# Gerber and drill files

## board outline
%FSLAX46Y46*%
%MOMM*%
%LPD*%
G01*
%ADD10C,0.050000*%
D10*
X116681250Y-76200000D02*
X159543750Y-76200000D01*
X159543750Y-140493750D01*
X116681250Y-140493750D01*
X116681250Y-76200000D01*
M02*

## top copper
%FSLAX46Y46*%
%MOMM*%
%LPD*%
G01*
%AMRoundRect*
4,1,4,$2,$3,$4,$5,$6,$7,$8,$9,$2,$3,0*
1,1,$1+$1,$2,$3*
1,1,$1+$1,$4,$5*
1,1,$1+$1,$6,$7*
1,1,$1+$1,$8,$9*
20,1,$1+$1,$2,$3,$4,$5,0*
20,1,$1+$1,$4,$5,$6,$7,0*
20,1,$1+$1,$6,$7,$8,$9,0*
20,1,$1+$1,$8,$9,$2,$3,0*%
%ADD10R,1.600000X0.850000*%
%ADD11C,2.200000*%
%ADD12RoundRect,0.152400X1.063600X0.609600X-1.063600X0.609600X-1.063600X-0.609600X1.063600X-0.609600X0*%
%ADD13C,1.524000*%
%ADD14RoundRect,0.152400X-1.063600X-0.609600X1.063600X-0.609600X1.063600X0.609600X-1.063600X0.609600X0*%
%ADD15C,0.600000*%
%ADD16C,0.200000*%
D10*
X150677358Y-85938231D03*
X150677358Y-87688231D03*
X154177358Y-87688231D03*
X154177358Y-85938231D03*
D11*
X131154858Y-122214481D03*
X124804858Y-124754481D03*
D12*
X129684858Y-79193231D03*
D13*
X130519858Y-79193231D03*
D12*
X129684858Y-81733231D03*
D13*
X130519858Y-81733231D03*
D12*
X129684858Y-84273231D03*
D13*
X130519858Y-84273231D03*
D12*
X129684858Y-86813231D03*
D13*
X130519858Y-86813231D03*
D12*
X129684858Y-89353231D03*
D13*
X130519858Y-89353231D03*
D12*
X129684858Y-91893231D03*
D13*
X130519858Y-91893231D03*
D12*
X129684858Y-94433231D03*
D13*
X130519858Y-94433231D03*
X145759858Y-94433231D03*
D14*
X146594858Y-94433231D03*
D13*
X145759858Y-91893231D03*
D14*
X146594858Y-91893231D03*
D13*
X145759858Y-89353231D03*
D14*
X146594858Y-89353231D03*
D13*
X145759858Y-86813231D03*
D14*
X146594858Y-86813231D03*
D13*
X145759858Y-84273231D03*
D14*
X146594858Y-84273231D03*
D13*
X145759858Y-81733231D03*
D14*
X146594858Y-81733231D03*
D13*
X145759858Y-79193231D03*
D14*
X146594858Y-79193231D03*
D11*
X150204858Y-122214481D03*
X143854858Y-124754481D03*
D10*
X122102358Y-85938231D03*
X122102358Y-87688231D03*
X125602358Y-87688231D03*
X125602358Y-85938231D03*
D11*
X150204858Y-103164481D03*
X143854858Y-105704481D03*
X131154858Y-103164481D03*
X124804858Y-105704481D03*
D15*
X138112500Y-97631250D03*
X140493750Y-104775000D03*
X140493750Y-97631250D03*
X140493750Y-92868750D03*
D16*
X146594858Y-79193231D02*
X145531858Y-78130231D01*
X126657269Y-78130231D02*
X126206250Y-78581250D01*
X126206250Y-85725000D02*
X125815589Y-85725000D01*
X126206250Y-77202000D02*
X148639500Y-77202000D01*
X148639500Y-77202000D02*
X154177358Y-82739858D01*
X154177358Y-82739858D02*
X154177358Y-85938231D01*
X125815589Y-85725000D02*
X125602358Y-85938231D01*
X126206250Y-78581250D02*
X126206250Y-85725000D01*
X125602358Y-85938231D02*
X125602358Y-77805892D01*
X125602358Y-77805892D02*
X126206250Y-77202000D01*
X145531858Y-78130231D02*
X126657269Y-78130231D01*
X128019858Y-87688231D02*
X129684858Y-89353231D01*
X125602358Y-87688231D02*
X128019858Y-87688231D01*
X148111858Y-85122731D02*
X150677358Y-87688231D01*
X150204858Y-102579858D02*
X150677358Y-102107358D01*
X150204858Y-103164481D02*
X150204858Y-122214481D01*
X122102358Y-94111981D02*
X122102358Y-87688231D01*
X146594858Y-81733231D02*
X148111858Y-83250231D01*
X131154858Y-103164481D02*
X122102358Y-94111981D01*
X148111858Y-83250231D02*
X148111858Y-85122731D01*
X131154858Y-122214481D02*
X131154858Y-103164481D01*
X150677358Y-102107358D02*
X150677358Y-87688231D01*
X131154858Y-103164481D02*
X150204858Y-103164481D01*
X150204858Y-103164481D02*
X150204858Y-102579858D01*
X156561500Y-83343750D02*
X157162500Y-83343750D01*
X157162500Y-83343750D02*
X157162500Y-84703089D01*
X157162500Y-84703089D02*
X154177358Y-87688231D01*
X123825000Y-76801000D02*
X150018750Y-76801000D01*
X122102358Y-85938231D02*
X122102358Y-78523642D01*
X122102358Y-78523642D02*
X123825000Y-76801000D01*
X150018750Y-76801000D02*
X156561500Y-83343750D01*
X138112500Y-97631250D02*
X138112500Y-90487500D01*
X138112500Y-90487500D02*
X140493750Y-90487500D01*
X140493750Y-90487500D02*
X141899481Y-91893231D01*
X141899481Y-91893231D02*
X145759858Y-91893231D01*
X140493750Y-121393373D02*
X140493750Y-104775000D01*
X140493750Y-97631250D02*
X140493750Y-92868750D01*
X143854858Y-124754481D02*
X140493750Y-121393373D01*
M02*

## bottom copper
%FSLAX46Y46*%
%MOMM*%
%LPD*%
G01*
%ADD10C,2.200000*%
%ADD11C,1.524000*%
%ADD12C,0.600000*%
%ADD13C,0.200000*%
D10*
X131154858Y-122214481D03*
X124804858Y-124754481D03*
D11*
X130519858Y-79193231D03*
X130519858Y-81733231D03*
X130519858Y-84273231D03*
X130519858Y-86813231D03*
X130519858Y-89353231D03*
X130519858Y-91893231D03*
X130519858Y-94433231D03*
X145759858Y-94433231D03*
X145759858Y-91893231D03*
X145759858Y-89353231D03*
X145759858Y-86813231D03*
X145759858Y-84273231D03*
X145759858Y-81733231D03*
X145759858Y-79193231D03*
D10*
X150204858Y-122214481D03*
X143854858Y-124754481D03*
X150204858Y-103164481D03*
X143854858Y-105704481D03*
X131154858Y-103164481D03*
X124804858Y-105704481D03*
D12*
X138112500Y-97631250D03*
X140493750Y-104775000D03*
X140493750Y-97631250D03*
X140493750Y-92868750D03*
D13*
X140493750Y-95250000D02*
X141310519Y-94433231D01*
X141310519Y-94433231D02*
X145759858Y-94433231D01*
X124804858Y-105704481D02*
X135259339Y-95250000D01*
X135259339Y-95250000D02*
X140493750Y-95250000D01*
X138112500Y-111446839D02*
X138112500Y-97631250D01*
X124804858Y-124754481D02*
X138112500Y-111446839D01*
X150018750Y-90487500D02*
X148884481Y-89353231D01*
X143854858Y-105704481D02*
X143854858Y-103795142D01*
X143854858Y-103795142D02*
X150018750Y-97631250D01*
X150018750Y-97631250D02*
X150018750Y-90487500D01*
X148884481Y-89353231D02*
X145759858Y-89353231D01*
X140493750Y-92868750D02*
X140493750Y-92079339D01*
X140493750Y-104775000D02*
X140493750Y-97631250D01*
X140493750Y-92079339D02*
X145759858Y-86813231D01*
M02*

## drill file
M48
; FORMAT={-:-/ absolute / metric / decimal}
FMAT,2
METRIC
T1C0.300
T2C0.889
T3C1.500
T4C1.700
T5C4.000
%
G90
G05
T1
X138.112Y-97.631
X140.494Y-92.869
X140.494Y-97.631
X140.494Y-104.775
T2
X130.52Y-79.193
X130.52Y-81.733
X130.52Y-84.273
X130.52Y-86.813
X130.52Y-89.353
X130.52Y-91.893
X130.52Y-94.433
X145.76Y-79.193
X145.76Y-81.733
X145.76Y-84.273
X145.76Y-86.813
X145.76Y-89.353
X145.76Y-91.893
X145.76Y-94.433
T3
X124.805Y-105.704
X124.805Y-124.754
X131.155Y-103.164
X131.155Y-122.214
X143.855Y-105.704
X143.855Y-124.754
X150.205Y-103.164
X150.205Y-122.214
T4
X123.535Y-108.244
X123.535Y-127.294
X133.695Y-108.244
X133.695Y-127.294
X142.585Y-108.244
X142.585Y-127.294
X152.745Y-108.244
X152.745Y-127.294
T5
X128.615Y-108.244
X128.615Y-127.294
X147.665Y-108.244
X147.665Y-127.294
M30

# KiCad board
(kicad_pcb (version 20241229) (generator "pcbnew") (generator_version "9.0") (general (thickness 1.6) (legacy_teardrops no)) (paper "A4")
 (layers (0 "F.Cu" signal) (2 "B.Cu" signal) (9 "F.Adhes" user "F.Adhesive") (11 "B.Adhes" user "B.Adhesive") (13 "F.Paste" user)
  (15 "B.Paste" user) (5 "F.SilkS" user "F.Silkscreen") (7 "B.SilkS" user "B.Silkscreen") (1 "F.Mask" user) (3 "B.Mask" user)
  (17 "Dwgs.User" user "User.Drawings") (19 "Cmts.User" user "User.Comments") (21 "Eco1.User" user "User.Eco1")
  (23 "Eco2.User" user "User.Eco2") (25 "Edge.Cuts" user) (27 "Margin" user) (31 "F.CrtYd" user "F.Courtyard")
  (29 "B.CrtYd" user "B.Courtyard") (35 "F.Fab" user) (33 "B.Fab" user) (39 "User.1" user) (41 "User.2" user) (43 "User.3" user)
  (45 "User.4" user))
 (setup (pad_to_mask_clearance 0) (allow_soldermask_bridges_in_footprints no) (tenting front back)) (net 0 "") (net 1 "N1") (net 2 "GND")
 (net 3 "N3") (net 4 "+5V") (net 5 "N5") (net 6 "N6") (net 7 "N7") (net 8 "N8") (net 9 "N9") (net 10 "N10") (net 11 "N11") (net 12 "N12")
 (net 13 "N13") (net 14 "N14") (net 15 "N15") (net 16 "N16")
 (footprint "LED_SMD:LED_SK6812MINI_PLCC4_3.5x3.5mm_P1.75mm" (layer "F.Cu") (at 152.427358 86.813231)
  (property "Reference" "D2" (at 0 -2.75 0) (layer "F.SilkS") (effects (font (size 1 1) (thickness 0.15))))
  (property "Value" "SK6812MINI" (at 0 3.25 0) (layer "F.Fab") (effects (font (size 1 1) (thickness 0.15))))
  (pad "1" smd rect (at -1.75 -0.875) (size 1.6 0.85) (layers "F.Cu" "F.Mask" "F.Paste") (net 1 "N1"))
  (pad "2" smd rect (at -1.75 0.875) (size 1.6 0.85) (layers "F.Cu" "F.Mask" "F.Paste") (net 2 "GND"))
  (pad "3" smd rect (at 1.75 0.875) (size 1.6 0.85) (layers "F.Cu" "F.Mask" "F.Paste") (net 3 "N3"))
  (pad "4" smd rect (at 1.75 -0.875) (size 1.6 0.85) (layers "F.Cu" "F.Mask" "F.Paste") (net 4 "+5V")))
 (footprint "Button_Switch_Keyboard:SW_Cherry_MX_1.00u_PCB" (layer "F.Cu") (at 131.154858 122.214481)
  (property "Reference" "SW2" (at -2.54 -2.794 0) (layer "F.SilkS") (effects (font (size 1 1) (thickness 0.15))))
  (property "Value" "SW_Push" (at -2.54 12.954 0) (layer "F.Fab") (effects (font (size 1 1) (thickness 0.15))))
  (pad "" np_thru_hole circle (at -7.62 5.08) (size 1.7 1.7) (drill 1.7) (layers "*.Cu" "*.Mask"))
  (pad "" np_thru_hole circle (at -2.54 5.08) (size 4 4) (drill 4) (layers "*.Cu" "*.Mask"))
  (pad "" np_thru_hole circle (at 2.54 5.08) (size 1.7 1.7) (drill 1.7) (layers "*.Cu" "*.Mask"))
  (pad "1" thru_hole circle (at 0 0) (size 2.2 2.2) (drill 1.5) (layers "*.Cu" "*.Mask") (remove_unused_layers no) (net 2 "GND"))
  (pad "2" thru_hole circle (at -6.35 2.54) (size 2.2 2.2) (drill 1.5) (layers "*.Cu" "*.Mask") (remove_unused_layers no) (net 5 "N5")))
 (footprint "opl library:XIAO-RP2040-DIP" (layer "F.Cu") (at 138.139858 86.813231)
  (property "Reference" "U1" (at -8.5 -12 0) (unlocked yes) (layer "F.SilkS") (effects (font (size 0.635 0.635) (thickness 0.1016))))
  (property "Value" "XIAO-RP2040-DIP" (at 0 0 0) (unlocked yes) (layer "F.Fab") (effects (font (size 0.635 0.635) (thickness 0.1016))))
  (pad "1" smd roundrect (at -8.455 -7.62 180) (size 2.432 1.524) (layers "F.Cu" "F.Mask") (roundrect_rratio 0.1) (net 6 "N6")
   (thermal_bridge_angle 45))
  (pad "1" thru_hole circle (at -7.62 -7.62 180) (size 1.524 1.524) (drill 0.889) (layers "*.Cu" "*.Mask") (remove_unused_layers no)
   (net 6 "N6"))
  (pad "2" smd roundrect (at -8.455 -5.08 180) (size 2.432 1.524) (layers "F.Cu" "F.Mask") (roundrect_rratio 0.1) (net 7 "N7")
   (thermal_bridge_angle 45))
  (pad "2" thru_hole circle (at -7.62 -5.08 180) (size 1.524 1.524) (drill 0.889) (layers "*.Cu" "*.Mask") (remove_unused_layers no)
   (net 7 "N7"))
  (pad "3" smd roundrect (at -8.455 -2.54 180) (size 2.432 1.524) (layers "F.Cu" "F.Mask") (roundrect_rratio 0.1) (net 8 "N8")
   (thermal_bridge_angle 45))
  (pad "3" thru_hole circle (at -7.62 -2.54 180) (size 1.524 1.524) (drill 0.889) (layers "*.Cu" "*.Mask") (remove_unused_layers no)
   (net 8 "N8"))
  (pad "4" smd roundrect (at -8.455 0 180) (size 2.432 1.524) (layers "F.Cu" "F.Mask") (roundrect_rratio 0.1) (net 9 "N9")
   (thermal_bridge_angle 45))
  (pad "4" thru_hole circle (at -7.62 0 180) (size 1.524 1.524) (drill 0.889) (layers "*.Cu" "*.Mask") (remove_unused_layers no)
   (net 9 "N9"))
  (pad "5" smd roundrect (at -8.455 2.54 180) (size 2.432 1.524) (layers "F.Cu" "F.Mask") (roundrect_rratio 0.1) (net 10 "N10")
   (thermal_bridge_angle 45))
  (pad "5" thru_hole circle (at -7.62 2.54 180) (size 1.524 1.524) (drill 0.889) (layers "*.Cu" "*.Mask") (remove_unused_layers no)
   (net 10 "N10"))
  (pad "6" smd roundrect (at -8.455 5.08 180) (size 2.432 1.524) (layers "F.Cu" "F.Mask") (roundrect_rratio 0.1) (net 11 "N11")
   (thermal_bridge_angle 45))
  (pad "6" thru_hole circle (at -7.62 5.08 180) (size 1.524 1.524) (drill 0.889) (layers "*.Cu" "*.Mask") (remove_unused_layers no)
   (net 11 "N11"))
  (pad "7" smd roundrect (at -8.455 7.62 180) (size 2.432 1.524) (layers "F.Cu" "F.Mask") (roundrect_rratio 0.1) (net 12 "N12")
   (thermal_bridge_angle 45))
  (pad "7" thru_hole circle (at -7.62 7.62 180) (size 1.524 1.524) (drill 0.889) (layers "*.Cu" "*.Mask") (remove_unused_layers no)
   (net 12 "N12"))
  (pad "8" thru_hole circle (at 7.62 7.62) (size 1.524 1.524) (drill 0.889) (layers "*.Cu" "*.Mask") (remove_unused_layers no)
   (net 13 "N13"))
  (pad "8" smd roundrect (at 8.455 7.62) (size 2.432 1.524) (layers "F.Cu" "F.Mask") (roundrect_rratio 0.1) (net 13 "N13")
   (thermal_bridge_angle 45))
  (pad "9" thru_hole circle (at 7.62 5.08) (size 1.524 1.524) (drill 0.889) (layers "*.Cu" "*.Mask") (remove_unused_layers no) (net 5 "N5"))
  (pad "9" smd roundrect (at 8.455 5.08) (size 2.432 1.524) (layers "F.Cu" "F.Mask") (roundrect_rratio 0.1) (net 5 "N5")
   (thermal_bridge_angle 45))
  (pad "10" thru_hole circle (at 7.62 2.54) (size 1.524 1.524) (drill 0.889) (layers "*.Cu" "*.Mask") (remove_unused_layers no)
   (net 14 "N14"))
  (pad "10" smd roundrect (at 8.455 2.54) (size 2.432 1.524) (layers "F.Cu" "F.Mask") (roundrect_rratio 0.1) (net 14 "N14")
   (thermal_bridge_angle 45))
  (pad "11" thru_hole circle (at 7.62 0) (size 1.524 1.524) (drill 0.889) (layers "*.Cu" "*.Mask") (remove_unused_layers no) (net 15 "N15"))
  (pad "11" smd roundrect (at 8.455 0) (size 2.432 1.524) (layers "F.Cu" "F.Mask") (roundrect_rratio 0.1) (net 15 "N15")
   (thermal_bridge_angle 45))
  (pad "12" thru_hole circle (at 7.62 -2.54) (size 1.524 1.524) (drill 0.889) (layers "*.Cu" "*.Mask") (remove_unused_layers no)
   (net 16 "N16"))
  (pad "12" smd roundrect (at 8.455 -2.54) (size 2.432 1.524) (layers "F.Cu" "F.Mask") (roundrect_rratio 0.1) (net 16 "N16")
   (thermal_bridge_angle 45))
  (pad "13" thru_hole circle (at 7.62 -5.08) (size 1.524 1.524) (drill 0.889) (layers "*.Cu" "*.Mask") (remove_unused_layers no)
   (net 2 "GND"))
  (pad "13" smd roundrect (at 8.455 -5.08) (size 2.432 1.524) (layers "F.Cu" "F.Mask") (roundrect_rratio 0.1) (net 2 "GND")
   (thermal_bridge_angle 45))
  (pad "14" thru_hole circle (at 7.62 -7.62) (size 1.524 1.524) (drill 0.889) (layers "*.Cu" "*.Mask") (remove_unused_layers no)
   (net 4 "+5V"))
  (pad "14" smd roundrect (at 8.455 -7.62) (size 2.432 1.524) (layers "F.Cu" "F.Mask") (roundrect_rratio 0.1) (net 4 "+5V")
   (thermal_bridge_angle 45)))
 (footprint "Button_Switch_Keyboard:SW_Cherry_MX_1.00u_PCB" (layer "F.Cu") (at 150.204858 122.214481)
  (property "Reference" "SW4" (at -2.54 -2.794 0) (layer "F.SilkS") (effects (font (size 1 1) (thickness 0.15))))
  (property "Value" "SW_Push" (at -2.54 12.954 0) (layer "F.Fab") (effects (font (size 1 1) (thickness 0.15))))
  (pad "" np_thru_hole circle (at -7.62 5.08) (size 1.7 1.7) (drill 1.7) (layers "*.Cu" "*.Mask"))
  (pad "" np_thru_hole circle (at -2.54 5.08) (size 4 4) (drill 4) (layers "*.Cu" "*.Mask"))
  (pad "" np_thru_hole circle (at 2.54 5.08) (size 1.7 1.7) (drill 1.7) (layers "*.Cu" "*.Mask"))
  (pad "1" thru_hole circle (at 0 0) (size 2.2 2.2) (drill 1.5) (layers "*.Cu" "*.Mask") (remove_unused_layers no) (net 2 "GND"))
  (pad "2" thru_hole circle (at -6.35 2.54) (size 2.2 2.2) (drill 1.5) (layers "*.Cu" "*.Mask") (remove_unused_layers no) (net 15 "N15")))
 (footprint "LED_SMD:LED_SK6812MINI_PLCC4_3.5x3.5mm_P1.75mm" (layer "F.Cu") (at 123.852358 86.813231)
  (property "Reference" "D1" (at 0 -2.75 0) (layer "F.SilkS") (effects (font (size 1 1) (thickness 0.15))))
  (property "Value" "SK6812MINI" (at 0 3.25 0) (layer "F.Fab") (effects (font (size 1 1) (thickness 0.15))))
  (pad "1" smd rect (at -1.75 -0.875) (size 1.6 0.85) (layers "F.Cu" "F.Mask" "F.Paste") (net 3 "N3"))
  (pad "2" smd rect (at -1.75 0.875) (size 1.6 0.85) (layers "F.Cu" "F.Mask" "F.Paste") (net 2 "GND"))
  (pad "3" smd rect (at 1.75 0.875) (size 1.6 0.85) (layers "F.Cu" "F.Mask" "F.Paste") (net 10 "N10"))
  (pad "4" smd rect (at 1.75 -0.875) (size 1.6 0.85) (layers "F.Cu" "F.Mask" "F.Paste") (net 4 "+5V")))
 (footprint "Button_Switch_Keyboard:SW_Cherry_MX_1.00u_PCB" (layer "F.Cu") (at 150.204858 103.164481)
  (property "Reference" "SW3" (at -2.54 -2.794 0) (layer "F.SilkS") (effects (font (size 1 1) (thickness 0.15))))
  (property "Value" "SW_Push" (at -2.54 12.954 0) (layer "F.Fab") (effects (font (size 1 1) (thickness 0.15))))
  (pad "" np_thru_hole circle (at -7.62 5.08) (size 1.7 1.7) (drill 1.7) (layers "*.Cu" "*.Mask"))
  (pad "" np_thru_hole circle (at -2.54 5.08) (size 4 4) (drill 4) (layers "*.Cu" "*.Mask"))
  (pad "" np_thru_hole circle (at 2.54 5.08) (size 1.7 1.7) (drill 1.7) (layers "*.Cu" "*.Mask"))
  (pad "1" thru_hole circle (at 0 0) (size 2.2 2.2) (drill 1.5) (layers "*.Cu" "*.Mask") (remove_unused_layers no) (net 2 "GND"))
  (pad "2" thru_hole circle (at -6.35 2.54) (size 2.2 2.2) (drill 1.5) (layers "*.Cu" "*.Mask") (remove_unused_layers no) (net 14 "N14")))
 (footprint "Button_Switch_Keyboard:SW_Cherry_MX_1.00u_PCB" (layer "F.Cu") (at 131.154858 103.164481)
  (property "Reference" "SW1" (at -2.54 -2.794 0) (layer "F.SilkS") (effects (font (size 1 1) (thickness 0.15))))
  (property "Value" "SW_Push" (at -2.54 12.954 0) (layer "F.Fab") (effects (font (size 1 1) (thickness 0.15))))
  (pad "" np_thru_hole circle (at -7.62 5.08) (size 1.7 1.7) (drill 1.7) (layers "*.Cu" "*.Mask"))
  (pad "" np_thru_hole circle (at -2.54 5.08) (size 4 4) (drill 4) (layers "*.Cu" "*.Mask"))
  (pad "" np_thru_hole circle (at 2.54 5.08) (size 1.7 1.7) (drill 1.7) (layers "*.Cu" "*.Mask"))
  (pad "1" thru_hole circle (at 0 0) (size 2.2 2.2) (drill 1.5) (layers "*.Cu" "*.Mask") (remove_unused_layers no) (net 2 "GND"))
  (pad "2" thru_hole circle (at -6.35 2.54) (size 2.2 2.2) (drill 1.5) (layers "*.Cu" "*.Mask") (remove_unused_layers no) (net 13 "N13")))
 (gr_rect (start 116.68125 76.2) (end 159.54375 140.49375) (stroke (width 0.05) (type default)) (fill no) (layer "Edge.Cuts"))
 (segment (start 146.594858 79.193231) (end 145.531858 78.130231) (width 0.2) (layer "F.Cu") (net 4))
 (segment (start 126.657269 78.130231) (end 126.20625 78.58125) (width 0.2) (layer "F.Cu") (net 4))
 (segment (start 126.20625 85.725) (end 125.815589 85.725) (width 0.2) (layer "F.Cu") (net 4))
 (segment (start 126.20625 77.202) (end 148.6395 77.202) (width 0.2) (layer "F.Cu") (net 4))
 (segment (start 148.6395 77.202) (end 154.177358 82.739858) (width 0.2) (layer "F.Cu") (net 4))
 (segment (start 154.177358 82.739858) (end 154.177358 85.938231) (width 0.2) (layer "F.Cu") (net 4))
 (segment (start 125.815589 85.725) (end 125.602358 85.938231) (width 0.2) (layer "F.Cu") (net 4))
 (segment (start 126.20625 78.58125) (end 126.20625 85.725) (width 0.2) (layer "F.Cu") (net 4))
 (segment (start 125.602358 85.938231) (end 125.602358 77.805892) (width 0.2) (layer "F.Cu") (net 4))
 (segment (start 125.602358 77.805892) (end 126.20625 77.202) (width 0.2) (layer "F.Cu") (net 4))
 (segment (start 145.531858 78.130231) (end 126.657269 78.130231) (width 0.2) (layer "F.Cu") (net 4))
 (segment (start 128.019858 87.688231) (end 129.684858 89.353231) (width 0.2) (layer "F.Cu") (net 10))
 (segment (start 125.602358 87.688231) (end 128.019858 87.688231) (width 0.2) (layer "F.Cu") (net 10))
 (segment (start 148.111858 85.122731) (end 150.677358 87.688231) (width 0.2) (layer "F.Cu") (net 2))
 (segment (start 150.204858 102.579858) (end 150.677358 102.107358) (width 0.2) (layer "F.Cu") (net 2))
 (segment (start 150.204858 103.164481) (end 150.204858 122.214481) (width 0.2) (layer "F.Cu") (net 2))
 (segment (start 122.102358 94.111981) (end 122.102358 87.688231) (width 0.2) (layer "F.Cu") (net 2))
 (segment (start 146.594858 81.733231) (end 148.111858 83.250231) (width 0.2) (layer "F.Cu") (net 2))
 (segment (start 131.154858 103.164481) (end 122.102358 94.111981) (width 0.2) (layer "F.Cu") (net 2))
 (segment (start 148.111858 83.250231) (end 148.111858 85.122731) (width 0.2) (layer "F.Cu") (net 2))
 (segment (start 131.154858 122.214481) (end 131.154858 103.164481) (width 0.2) (layer "F.Cu") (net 2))
 (segment (start 150.677358 102.107358) (end 150.677358 87.688231) (width 0.2) (layer "F.Cu") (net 2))
 (segment (start 131.154858 103.164481) (end 150.204858 103.164481) (width 0.2) (layer "F.Cu") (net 2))
 (segment (start 150.204858 103.164481) (end 150.204858 102.579858) (width 0.2) (layer "F.Cu") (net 2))
 (segment (start 156.5615 83.34375) (end 157.1625 83.34375) (width 0.2) (layer "F.Cu") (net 3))
 (segment (start 157.1625 83.34375) (end 157.1625 84.703089) (width 0.2) (layer "F.Cu") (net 3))
 (segment (start 157.1625 84.703089) (end 154.177358 87.688231) (width 0.2) (layer "F.Cu") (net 3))
 (segment (start 123.825 76.801) (end 150.01875 76.801) (width 0.2) (layer "F.Cu") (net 3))
 (segment (start 122.102358 85.938231) (end 122.102358 78.523642) (width 0.2) (layer "F.Cu") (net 3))
 (segment (start 122.102358 78.523642) (end 123.825 76.801) (width 0.2) (layer "F.Cu") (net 3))
 (segment (start 150.01875 76.801) (end 156.5615 83.34375) (width 0.2) (layer "F.Cu") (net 3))
 (segment (start 140.49375 95.25) (end 141.310519 94.433231) (width 0.2) (layer "B.Cu") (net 13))
 (segment (start 141.310519 94.433231) (end 145.759858 94.433231) (width 0.2) (layer "B.Cu") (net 13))
 (segment (start 124.804858 105.704481) (end 135.259339 95.25) (width 0.2) (layer "B.Cu") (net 13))
 (segment (start 135.259339 95.25) (end 140.49375 95.25) (width 0.2) (layer "B.Cu") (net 13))
 (segment (start 138.1125 97.63125) (end 138.1125 90.4875) (width 0.2) (layer "F.Cu") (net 5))
 (segment (start 138.1125 90.4875) (end 140.49375 90.4875) (width 0.2) (layer "F.Cu") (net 5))
 (segment (start 140.49375 90.4875) (end 141.899481 91.893231) (width 0.2) (layer "F.Cu") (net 5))
 (segment (start 141.899481 91.893231) (end 145.759858 91.893231) (width 0.2) (layer "F.Cu") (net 5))
 (via (at 138.1125 97.63125) (size 0.6) (drill 0.3) (layers "F.Cu" "B.Cu") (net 5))
 (segment (start 138.1125 111.446839) (end 138.1125 97.63125) (width 0.2) (layer "B.Cu") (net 5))
 (segment (start 124.804858 124.754481) (end 138.1125 111.446839) (width 0.2) (layer "B.Cu") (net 5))
 (segment (start 150.01875 90.4875) (end 148.884481 89.353231) (width 0.2) (layer "B.Cu") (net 14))
 (segment (start 143.854858 105.704481) (end 143.854858 103.795142) (width 0.2) (layer "B.Cu") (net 14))
 (segment (start 143.854858 103.795142) (end 150.01875 97.63125) (width 0.2) (layer "B.Cu") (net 14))
 (segment (start 150.01875 97.63125) (end 150.01875 90.4875) (width 0.2) (layer "B.Cu") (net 14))
 (segment (start 148.884481 89.353231) (end 145.759858 89.353231) (width 0.2) (layer "B.Cu") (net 14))
 (segment (start 140.49375 121.393373) (end 140.49375 104.775) (width 0.2) (layer "F.Cu") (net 15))
 (segment (start 140.49375 97.63125) (end 140.49375 92.86875) (width 0.2) (layer "F.Cu") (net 15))
 (segment (start 143.854858 124.754481) (end 140.49375 121.393373) (width 0.2) (layer "F.Cu") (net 15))
 (via (at 140.49375 104.775) (size 0.6) (drill 0.3) (layers "F.Cu" "B.Cu") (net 15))
 (via (at 140.49375 97.63125) (size 0.6) (drill 0.3) (layers "F.Cu" "B.Cu") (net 15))
 (via (at 140.49375 92.86875) (size 0.6) (drill 0.3) (layers "F.Cu" "B.Cu") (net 15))
 (segment (start 140.49375 92.86875) (end 140.49375 92.079339) (width 0.2) (layer "B.Cu") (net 15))
 (segment (start 140.49375 104.775) (end 140.49375 97.63125) (width 0.2) (layer "B.Cu") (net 15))
 (segment (start 140.49375 92.079339) (end 145.759858 86.813231) (width 0.2) (layer "B.Cu") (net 15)))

